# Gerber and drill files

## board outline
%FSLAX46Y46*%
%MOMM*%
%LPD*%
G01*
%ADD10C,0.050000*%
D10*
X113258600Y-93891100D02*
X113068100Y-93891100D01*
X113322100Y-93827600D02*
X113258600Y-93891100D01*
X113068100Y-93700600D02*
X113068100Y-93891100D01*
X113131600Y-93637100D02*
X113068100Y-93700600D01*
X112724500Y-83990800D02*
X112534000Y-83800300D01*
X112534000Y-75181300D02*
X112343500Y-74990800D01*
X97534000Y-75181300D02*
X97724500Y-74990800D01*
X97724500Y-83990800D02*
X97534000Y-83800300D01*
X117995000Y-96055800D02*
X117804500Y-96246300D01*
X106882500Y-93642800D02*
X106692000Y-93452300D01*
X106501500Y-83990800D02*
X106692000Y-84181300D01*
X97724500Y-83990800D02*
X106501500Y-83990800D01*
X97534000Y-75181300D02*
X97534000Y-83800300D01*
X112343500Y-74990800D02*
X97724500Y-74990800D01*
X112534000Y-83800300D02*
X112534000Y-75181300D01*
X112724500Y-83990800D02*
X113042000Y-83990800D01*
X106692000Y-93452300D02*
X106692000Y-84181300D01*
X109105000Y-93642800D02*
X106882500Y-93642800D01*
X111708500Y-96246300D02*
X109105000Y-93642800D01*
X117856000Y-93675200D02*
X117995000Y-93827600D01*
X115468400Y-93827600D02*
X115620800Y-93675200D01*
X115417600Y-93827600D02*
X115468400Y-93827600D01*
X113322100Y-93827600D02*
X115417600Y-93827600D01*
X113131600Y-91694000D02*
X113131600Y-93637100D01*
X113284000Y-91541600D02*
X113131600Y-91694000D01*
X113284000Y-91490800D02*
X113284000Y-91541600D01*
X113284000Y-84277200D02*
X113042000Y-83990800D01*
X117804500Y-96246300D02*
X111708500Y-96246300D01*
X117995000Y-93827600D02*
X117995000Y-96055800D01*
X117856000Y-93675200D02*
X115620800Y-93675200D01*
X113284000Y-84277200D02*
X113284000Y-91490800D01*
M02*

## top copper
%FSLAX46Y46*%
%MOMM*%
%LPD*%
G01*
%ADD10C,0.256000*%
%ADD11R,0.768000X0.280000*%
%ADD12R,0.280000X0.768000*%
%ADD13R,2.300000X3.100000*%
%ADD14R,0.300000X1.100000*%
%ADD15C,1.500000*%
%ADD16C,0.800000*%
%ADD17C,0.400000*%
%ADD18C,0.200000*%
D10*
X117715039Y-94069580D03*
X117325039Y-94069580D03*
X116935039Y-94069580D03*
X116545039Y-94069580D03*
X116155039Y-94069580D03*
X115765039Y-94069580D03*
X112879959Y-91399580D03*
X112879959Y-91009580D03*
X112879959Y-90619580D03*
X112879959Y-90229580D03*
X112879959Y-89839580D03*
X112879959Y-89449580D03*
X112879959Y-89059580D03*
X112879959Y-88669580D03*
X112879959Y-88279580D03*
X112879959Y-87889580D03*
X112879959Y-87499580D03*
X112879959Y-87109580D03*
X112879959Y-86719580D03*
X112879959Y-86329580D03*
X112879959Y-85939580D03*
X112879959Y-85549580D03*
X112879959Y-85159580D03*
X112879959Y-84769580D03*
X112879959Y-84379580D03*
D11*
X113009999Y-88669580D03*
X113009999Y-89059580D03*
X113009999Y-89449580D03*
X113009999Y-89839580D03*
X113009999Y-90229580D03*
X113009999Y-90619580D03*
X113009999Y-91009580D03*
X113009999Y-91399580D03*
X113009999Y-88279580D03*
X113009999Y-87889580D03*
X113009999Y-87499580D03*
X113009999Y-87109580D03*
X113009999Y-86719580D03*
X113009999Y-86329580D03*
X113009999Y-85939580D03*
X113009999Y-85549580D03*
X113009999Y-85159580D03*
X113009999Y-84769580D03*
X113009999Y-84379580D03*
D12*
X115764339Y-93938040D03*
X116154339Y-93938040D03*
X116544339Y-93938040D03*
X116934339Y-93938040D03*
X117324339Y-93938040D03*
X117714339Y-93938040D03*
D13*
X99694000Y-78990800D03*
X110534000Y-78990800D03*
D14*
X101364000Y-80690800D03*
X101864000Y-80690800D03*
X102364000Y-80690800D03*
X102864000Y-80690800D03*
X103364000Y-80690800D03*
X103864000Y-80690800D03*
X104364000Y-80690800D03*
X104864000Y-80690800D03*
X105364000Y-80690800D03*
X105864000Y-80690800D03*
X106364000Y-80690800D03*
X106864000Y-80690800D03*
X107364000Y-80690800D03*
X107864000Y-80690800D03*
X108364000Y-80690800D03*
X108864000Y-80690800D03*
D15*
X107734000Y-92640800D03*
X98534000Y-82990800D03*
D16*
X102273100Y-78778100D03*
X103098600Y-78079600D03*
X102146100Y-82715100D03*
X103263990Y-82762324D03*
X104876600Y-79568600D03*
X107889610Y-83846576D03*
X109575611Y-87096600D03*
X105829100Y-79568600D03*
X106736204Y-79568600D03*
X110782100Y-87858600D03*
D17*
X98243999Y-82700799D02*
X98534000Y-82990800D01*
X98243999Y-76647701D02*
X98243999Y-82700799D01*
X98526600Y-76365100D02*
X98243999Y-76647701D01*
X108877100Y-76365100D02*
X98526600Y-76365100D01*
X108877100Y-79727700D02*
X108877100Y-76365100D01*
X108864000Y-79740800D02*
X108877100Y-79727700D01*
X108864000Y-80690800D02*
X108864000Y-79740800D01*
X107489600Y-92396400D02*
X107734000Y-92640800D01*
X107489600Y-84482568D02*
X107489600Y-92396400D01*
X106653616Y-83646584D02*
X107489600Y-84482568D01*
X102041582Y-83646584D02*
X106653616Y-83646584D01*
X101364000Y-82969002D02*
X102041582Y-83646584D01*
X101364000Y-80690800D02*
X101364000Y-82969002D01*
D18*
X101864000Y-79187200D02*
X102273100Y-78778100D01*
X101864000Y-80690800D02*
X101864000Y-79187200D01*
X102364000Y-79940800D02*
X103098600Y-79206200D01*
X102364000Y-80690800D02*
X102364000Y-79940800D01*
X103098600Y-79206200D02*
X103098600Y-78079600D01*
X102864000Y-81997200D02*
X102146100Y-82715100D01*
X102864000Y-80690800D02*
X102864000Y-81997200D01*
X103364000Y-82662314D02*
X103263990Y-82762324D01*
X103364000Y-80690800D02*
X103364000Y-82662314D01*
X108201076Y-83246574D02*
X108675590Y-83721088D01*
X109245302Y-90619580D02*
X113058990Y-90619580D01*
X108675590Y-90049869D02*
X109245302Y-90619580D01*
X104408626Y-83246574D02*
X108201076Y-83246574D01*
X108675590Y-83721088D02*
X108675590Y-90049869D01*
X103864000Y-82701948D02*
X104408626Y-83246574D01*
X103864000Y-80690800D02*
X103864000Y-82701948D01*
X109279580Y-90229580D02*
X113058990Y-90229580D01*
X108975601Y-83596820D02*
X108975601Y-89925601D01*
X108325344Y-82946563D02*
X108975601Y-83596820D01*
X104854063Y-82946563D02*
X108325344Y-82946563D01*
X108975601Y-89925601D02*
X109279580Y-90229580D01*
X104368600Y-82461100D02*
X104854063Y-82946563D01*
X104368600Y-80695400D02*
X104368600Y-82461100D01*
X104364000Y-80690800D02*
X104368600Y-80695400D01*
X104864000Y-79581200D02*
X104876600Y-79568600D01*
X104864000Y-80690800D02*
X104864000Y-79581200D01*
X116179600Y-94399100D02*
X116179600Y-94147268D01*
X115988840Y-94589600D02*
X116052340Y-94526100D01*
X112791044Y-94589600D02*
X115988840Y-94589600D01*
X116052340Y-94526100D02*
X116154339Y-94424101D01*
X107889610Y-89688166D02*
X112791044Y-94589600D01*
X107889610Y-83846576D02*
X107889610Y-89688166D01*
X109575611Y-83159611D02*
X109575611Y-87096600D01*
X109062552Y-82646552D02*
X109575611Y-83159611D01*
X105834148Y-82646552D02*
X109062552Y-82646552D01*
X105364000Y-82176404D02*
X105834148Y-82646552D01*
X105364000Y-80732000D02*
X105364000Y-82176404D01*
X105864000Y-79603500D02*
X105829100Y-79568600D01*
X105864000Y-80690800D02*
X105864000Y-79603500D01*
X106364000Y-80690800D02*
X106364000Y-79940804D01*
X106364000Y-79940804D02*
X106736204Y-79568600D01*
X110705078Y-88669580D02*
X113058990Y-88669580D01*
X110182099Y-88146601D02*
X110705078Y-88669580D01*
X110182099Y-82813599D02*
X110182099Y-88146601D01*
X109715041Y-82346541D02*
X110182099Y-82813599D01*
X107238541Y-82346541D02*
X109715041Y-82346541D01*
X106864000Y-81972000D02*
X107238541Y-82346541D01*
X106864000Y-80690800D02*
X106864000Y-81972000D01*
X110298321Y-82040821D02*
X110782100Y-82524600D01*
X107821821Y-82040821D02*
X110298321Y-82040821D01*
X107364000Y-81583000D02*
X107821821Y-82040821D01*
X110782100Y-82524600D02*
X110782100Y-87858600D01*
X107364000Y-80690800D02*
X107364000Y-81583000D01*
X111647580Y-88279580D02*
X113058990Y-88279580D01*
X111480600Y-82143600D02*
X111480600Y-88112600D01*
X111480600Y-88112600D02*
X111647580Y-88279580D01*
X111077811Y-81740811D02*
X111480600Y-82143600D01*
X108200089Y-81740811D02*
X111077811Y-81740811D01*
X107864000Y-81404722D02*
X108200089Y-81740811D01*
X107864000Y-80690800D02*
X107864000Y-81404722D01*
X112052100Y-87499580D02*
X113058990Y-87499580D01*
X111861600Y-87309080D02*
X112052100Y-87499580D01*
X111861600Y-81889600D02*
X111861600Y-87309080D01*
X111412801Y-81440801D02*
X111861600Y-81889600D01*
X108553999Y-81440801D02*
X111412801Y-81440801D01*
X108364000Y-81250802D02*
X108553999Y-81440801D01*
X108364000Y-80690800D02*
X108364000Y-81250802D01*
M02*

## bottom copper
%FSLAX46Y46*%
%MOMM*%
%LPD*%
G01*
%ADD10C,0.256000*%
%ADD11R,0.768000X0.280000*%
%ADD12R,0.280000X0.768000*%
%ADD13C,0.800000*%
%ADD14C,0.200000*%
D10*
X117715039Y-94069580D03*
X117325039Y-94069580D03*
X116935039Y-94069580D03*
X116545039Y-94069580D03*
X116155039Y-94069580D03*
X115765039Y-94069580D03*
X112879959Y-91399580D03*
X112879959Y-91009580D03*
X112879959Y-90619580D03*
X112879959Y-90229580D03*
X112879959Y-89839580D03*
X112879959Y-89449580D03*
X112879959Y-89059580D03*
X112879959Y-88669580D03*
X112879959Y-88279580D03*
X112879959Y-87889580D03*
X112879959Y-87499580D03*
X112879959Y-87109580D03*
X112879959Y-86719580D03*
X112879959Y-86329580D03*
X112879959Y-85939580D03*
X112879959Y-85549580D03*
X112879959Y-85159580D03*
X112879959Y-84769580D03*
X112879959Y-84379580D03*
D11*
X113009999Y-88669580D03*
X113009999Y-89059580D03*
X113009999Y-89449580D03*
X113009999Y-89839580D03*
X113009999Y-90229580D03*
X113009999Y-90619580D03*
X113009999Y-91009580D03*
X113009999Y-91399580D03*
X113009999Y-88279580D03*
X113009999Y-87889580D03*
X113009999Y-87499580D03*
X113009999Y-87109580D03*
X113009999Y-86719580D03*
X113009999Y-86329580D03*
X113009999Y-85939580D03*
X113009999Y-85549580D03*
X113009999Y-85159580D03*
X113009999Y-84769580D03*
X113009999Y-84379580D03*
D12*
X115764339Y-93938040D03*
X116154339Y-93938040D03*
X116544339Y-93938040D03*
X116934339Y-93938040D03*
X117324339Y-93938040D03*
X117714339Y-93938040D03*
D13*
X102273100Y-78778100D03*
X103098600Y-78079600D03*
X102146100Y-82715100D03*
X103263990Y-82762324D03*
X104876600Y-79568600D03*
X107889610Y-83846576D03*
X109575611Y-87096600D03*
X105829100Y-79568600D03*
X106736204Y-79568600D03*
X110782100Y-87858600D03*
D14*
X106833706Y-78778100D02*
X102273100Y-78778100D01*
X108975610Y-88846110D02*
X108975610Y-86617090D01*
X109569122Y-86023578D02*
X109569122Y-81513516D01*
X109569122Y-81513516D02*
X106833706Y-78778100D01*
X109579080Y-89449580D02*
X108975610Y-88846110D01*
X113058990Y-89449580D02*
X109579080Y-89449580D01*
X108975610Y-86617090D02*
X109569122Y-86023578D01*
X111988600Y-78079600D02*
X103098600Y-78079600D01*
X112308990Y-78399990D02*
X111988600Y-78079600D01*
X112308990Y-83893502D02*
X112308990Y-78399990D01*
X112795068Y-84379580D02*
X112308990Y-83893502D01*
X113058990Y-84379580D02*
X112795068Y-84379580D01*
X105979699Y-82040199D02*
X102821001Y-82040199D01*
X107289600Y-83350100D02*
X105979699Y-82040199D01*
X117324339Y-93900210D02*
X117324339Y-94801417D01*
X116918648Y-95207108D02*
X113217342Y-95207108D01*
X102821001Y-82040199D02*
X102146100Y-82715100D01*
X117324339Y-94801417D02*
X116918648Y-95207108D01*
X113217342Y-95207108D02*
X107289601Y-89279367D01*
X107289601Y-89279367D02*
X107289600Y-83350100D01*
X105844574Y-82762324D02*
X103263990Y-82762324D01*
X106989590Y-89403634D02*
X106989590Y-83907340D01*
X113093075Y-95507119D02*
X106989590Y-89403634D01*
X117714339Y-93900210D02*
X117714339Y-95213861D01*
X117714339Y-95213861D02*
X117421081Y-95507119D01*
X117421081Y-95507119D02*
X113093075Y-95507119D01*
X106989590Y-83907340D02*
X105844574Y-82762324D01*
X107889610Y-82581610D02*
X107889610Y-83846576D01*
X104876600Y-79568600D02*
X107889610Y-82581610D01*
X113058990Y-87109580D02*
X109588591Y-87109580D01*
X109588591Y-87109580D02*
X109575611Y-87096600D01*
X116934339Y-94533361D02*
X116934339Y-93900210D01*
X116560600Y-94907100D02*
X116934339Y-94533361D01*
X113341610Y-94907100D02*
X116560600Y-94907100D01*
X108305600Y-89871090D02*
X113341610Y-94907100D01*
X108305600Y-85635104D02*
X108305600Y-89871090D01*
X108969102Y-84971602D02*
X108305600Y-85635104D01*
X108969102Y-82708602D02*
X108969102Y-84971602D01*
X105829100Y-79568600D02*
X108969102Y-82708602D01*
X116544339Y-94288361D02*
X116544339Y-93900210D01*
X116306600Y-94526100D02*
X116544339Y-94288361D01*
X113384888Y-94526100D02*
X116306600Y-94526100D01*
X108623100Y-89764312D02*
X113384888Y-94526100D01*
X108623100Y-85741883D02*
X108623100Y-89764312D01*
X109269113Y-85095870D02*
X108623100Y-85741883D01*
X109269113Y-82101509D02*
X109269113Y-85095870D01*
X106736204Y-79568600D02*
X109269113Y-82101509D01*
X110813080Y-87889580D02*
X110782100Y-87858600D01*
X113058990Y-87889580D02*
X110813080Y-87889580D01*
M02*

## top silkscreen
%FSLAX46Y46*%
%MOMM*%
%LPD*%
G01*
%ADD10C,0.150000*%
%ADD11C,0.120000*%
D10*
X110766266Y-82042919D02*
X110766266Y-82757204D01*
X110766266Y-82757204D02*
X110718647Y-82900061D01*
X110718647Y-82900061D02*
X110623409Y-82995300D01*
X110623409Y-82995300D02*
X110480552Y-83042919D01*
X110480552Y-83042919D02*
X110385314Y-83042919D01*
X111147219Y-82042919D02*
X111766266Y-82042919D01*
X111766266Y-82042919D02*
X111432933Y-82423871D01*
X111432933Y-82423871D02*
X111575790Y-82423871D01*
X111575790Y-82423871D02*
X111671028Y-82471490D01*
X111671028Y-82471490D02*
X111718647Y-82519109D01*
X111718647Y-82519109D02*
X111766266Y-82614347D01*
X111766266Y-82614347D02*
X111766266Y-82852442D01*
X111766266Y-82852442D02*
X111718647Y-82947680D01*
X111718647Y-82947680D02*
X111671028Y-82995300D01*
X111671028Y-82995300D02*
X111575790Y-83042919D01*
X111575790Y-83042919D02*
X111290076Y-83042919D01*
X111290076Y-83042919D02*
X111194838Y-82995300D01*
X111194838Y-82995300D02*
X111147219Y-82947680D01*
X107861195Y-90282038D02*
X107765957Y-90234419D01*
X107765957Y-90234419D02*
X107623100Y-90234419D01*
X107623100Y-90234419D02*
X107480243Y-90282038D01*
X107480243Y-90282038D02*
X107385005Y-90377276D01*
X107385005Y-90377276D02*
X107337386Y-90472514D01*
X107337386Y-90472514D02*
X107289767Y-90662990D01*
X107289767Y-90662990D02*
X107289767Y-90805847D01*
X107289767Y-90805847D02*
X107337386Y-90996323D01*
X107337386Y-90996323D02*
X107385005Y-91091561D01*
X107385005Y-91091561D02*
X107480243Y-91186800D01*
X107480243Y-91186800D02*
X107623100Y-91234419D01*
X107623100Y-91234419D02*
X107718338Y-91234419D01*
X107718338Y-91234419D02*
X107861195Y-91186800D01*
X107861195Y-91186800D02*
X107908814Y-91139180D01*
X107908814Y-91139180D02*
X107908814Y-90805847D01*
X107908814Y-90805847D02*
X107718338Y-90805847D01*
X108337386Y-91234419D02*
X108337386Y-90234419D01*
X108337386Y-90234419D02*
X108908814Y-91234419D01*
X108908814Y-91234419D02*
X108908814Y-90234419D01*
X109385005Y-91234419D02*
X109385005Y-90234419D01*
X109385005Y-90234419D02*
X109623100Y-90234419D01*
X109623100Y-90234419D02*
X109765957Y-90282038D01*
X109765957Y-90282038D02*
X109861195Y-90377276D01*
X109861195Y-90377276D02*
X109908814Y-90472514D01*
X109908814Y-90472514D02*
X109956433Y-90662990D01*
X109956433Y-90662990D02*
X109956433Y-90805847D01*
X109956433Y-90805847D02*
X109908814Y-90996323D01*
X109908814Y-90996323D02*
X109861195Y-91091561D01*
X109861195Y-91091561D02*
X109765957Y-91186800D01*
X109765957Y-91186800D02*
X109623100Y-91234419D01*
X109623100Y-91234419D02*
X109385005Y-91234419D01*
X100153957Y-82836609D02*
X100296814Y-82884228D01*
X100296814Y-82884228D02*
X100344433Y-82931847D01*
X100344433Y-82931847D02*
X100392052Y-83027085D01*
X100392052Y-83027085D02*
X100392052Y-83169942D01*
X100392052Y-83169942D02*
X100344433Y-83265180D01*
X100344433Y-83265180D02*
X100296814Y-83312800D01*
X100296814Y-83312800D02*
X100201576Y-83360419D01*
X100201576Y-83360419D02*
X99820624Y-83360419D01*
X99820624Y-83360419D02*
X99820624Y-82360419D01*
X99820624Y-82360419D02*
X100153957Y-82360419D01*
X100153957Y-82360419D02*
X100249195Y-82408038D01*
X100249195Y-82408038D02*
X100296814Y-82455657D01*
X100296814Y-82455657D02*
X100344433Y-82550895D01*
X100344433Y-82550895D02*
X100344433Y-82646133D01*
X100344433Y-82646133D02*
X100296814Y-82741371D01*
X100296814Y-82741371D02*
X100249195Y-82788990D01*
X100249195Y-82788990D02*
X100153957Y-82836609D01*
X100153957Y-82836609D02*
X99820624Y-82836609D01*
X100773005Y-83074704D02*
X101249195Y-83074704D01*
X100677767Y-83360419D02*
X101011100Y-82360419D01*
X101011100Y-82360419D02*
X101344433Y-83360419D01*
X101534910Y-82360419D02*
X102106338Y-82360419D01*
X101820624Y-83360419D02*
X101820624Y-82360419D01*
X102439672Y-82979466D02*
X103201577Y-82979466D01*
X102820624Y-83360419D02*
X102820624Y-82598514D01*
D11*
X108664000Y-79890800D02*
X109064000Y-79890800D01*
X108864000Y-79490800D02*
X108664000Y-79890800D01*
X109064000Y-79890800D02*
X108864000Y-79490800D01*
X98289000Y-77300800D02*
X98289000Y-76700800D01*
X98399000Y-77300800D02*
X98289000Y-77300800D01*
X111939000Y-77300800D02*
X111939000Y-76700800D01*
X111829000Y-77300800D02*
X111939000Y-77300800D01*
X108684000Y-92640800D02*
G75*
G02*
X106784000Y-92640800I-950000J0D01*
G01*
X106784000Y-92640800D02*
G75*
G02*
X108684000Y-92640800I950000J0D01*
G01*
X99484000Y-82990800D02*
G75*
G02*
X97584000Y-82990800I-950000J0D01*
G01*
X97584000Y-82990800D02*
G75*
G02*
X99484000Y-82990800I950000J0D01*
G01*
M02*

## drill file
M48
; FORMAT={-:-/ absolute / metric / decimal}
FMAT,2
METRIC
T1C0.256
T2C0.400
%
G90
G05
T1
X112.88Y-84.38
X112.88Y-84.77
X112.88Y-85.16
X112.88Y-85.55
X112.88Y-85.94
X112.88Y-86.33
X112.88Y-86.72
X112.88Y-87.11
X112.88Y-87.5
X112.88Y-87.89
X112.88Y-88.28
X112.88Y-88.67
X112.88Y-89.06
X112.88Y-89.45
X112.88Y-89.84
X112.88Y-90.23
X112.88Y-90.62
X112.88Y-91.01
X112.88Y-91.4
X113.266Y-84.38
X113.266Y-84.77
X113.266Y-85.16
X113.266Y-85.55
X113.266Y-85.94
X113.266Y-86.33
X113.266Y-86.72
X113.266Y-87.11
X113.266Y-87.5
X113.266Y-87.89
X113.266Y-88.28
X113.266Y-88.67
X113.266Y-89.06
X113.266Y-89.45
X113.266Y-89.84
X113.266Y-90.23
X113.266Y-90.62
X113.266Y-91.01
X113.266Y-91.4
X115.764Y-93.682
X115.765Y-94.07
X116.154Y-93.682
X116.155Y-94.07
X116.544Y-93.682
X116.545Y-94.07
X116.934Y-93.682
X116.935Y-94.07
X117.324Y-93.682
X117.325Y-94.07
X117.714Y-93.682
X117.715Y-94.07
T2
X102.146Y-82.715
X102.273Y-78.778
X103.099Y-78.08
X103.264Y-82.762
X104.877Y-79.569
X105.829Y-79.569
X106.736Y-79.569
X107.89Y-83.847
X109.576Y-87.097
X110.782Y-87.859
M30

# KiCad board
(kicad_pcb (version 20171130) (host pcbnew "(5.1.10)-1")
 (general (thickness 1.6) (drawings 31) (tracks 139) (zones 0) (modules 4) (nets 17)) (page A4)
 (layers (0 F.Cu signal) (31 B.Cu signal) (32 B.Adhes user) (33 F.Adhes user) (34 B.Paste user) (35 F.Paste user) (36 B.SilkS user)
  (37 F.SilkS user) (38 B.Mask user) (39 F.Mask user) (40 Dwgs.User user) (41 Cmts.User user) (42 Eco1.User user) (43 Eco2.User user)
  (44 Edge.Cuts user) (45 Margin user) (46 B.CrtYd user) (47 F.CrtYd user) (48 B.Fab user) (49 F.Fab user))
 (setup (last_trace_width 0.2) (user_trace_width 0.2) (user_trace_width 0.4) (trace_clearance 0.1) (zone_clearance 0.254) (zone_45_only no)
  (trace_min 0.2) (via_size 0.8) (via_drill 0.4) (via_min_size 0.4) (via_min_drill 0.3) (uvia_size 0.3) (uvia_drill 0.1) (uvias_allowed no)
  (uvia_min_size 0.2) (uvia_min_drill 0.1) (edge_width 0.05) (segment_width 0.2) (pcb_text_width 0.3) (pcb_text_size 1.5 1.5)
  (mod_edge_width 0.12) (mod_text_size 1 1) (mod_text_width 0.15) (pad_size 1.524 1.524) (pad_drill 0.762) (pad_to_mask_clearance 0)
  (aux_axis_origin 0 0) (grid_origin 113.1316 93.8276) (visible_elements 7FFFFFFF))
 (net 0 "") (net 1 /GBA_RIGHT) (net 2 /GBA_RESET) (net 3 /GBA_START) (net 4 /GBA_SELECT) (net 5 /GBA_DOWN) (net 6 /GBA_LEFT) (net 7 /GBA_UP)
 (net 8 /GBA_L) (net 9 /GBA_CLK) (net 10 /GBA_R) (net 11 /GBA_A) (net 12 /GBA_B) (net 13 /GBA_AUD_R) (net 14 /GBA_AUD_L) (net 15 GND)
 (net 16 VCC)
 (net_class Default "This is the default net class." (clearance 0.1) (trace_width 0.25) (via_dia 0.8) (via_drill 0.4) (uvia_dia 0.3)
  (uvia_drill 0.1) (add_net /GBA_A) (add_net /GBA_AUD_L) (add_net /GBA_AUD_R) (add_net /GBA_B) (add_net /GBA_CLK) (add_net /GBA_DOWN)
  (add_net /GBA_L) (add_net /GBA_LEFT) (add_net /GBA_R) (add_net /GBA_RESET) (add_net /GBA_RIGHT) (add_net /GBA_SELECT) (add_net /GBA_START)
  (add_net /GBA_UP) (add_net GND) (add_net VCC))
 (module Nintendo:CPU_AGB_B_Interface (layer F.Cu) (at 115.759959 89.84808)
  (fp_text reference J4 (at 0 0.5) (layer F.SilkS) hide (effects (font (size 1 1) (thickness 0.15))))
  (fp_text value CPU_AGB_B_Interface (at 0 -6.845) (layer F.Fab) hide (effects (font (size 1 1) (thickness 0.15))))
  (pad 0 thru_hole circle (at 1.95508 4.2215) (size 0.256 0.256) (drill 0.256) (layers *.Cu *.Mask))
  (pad 0 thru_hole circle (at 1.56508 4.2215) (size 0.256 0.256) (drill 0.256) (layers *.Cu *.Mask))
  (pad 0 thru_hole circle (at 1.17508 4.2215) (size 0.256 0.256) (drill 0.256) (layers *.Cu *.Mask))
  (pad 0 thru_hole circle (at 0.78508 4.2215) (size 0.256 0.256) (drill 0.256) (layers *.Cu *.Mask))
  (pad 0 thru_hole circle (at 0.39508 4.2215) (size 0.256 0.256) (drill 0.256) (layers *.Cu *.Mask))
  (pad 0 thru_hole circle (at 0.00508 4.2215) (size 0.256 0.256) (drill 0.256) (layers *.Cu *.Mask))
  (pad 0 thru_hole circle (at -2.88 1.5515) (size 0.256 0.256) (drill 0.256) (layers *.Cu *.Mask))
  (pad 0 thru_hole circle (at -2.88 1.1615) (size 0.256 0.256) (drill 0.256) (layers *.Cu *.Mask))
  (pad 0 thru_hole circle (at -2.88 0.7715) (size 0.256 0.256) (drill 0.256) (layers *.Cu *.Mask))
  (pad 0 thru_hole circle (at -2.88 0.3815) (size 0.256 0.256) (drill 0.256) (layers *.Cu *.Mask))
  (pad 0 thru_hole circle (at -2.88 -0.0085) (size 0.256 0.256) (drill 0.256) (layers *.Cu *.Mask))
  (pad 0 thru_hole circle (at -2.88 -0.3985) (size 0.256 0.256) (drill 0.256) (layers *.Cu *.Mask))
  (pad 0 thru_hole circle (at -2.88 -0.7885) (size 0.256 0.256) (drill 0.256) (layers *.Cu *.Mask))
  (pad 0 thru_hole circle (at -2.88 -1.1785) (size 0.256 0.256) (drill 0.256) (layers *.Cu *.Mask))
  (pad 0 thru_hole circle (at -2.88 -1.5685) (size 0.256 0.256) (drill 0.256) (layers *.Cu *.Mask))
  (pad 0 thru_hole circle (at -2.88 -1.9585) (size 0.256 0.256) (drill 0.256) (layers *.Cu *.Mask))
  (pad 0 thru_hole circle (at -2.88 -2.3485) (size 0.256 0.256) (drill 0.256) (layers *.Cu *.Mask))
  (pad 0 thru_hole circle (at -2.88 -2.7385) (size 0.256 0.256) (drill 0.256) (layers *.Cu *.Mask))
  (pad 0 thru_hole circle (at -2.88 -3.1285) (size 0.256 0.256) (drill 0.256) (layers *.Cu *.Mask))
  (pad 0 thru_hole circle (at -2.88 -3.5185) (size 0.256 0.256) (drill 0.256) (layers *.Cu *.Mask))
  (pad 0 thru_hole circle (at -2.88 -3.9085) (size 0.256 0.256) (drill 0.256) (layers *.Cu *.Mask))
  (pad 0 thru_hole circle (at -2.88 -4.2985) (size 0.256 0.256) (drill 0.256) (layers *.Cu *.Mask))
  (pad 0 thru_hole circle (at -2.88 -4.6885) (size 0.256 0.256) (drill 0.256) (layers *.Cu *.Mask))
  (pad 0 thru_hole circle (at -2.88 -5.0785) (size 0.256 0.256) (drill 0.256) (layers *.Cu *.Mask))
  (pad 0 thru_hole circle (at -2.88 -5.4685) (size 0.256 0.256) (drill 0.256) (layers *.Cu *.Mask))
  (pad 149 thru_hole rect (at -2.49396 -1.1785) (size 0.768 0.28) (drill 0.256 (offset -0.256 0)) (layers *.Cu *.Mask) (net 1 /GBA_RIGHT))
  (pad 150 thru_hole rect (at -2.49396 -0.7885) (size 0.768 0.28) (drill 0.256 (offset -0.256 0)) (layers *.Cu *.Mask))
  (pad 151 thru_hole rect (at -2.49396 -0.3985) (size 0.768 0.28) (drill 0.256 (offset -0.256 0)) (layers *.Cu *.Mask) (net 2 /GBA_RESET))
  (pad 152 thru_hole rect (at -2.49396 -0.0085) (size 0.768 0.28) (drill 0.256 (offset -0.256 0)) (layers *.Cu *.Mask))
  (pad 153 thru_hole rect (at -2.49396 0.3815) (size 0.768 0.28) (drill 0.256 (offset -0.256 0)) (layers *.Cu *.Mask) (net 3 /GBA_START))
  (pad 154 thru_hole rect (at -2.49396 0.7715) (size 0.768 0.28) (drill 0.256 (offset -0.256 0)) (layers *.Cu *.Mask) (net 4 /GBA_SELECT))
  (pad 155 thru_hole rect (at -2.49396 1.1615) (size 0.768 0.28) (drill 0.256 (offset -0.256 0)) (layers *.Cu *.Mask))
  (pad 156 thru_hole rect (at -2.49396 1.5515) (size 0.768 0.28) (drill 0.256 (offset -0.256 0)) (layers *.Cu *.Mask))
  (pad 148 thru_hole rect (at -2.49396 -1.5685) (size 0.768 0.28) (drill 0.256 (offset -0.256 0)) (layers *.Cu *.Mask) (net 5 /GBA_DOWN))
  (pad 147 thru_hole rect (at -2.49396 -1.9585) (size 0.768 0.28) (drill 0.256 (offset -0.256 0)) (layers *.Cu *.Mask) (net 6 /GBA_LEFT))
  (pad 146 thru_hole rect (at -2.49396 -2.3485) (size 0.768 0.28) (drill 0.256 (offset -0.256 0)) (layers *.Cu *.Mask) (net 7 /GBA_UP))
  (pad 145 thru_hole rect (at -2.49396 -2.7385) (size 0.768 0.28) (drill 0.256 (offset -0.256 0)) (layers *.Cu *.Mask) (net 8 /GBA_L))
  (pad 144 thru_hole rect (at -2.49396 -3.1285) (size 0.768 0.28) (drill 0.256 (offset -0.256 0)) (layers *.Cu *.Mask))
  (pad 143 thru_hole rect (at -2.49396 -3.5185) (size 0.768 0.28) (drill 0.256 (offset -0.256 0)) (layers *.Cu *.Mask))
  (pad 142 thru_hole rect (at -2.49396 -3.9085) (size 0.768 0.28) (drill 0.256 (offset -0.256 0)) (layers *.Cu *.Mask))
  (pad 141 thru_hole rect (at -2.49396 -4.2985) (size 0.768 0.28) (drill 0.256 (offset -0.256 0)) (layers *.Cu *.Mask))
  (pad 140 thru_hole rect (at -2.49396 -4.6885) (size 0.768 0.28) (drill 0.256 (offset -0.256 0)) (layers *.Cu *.Mask))
  (pad 139 thru_hole rect (at -2.49396 -5.0785) (size 0.768 0.28) (drill 0.256 (offset -0.256 0)) (layers *.Cu *.Mask))
  (pad 138 thru_hole rect (at -2.49396 -5.4685) (size 0.768 0.28) (drill 0.256 (offset -0.256 0)) (layers *.Cu *.Mask) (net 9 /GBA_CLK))
  (pad 1 thru_hole rect (at 0.00438 3.83396 90) (size 0.768 0.28) (drill 0.256 (offset -0.256 0)) (layers *.Cu *.Mask))
  (pad 2 thru_hole rect (at 0.39438 3.83396 90) (size 0.768 0.28) (drill 0.256 (offset -0.256 0)) (layers *.Cu *.Mask) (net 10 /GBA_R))
  (pad 3 thru_hole rect (at 0.78438 3.83396 90) (size 0.768 0.28) (drill 0.256 (offset -0.256 0)) (layers *.Cu *.Mask) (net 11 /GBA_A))
  (pad 4 thru_hole rect (at 1.17438 3.83396 90) (size 0.768 0.28) (drill 0.256 (offset -0.256 0)) (layers *.Cu *.Mask) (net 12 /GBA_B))
  (pad 5 thru_hole rect (at 1.56438 3.83396 90) (size 0.768 0.28) (drill 0.256 (offset -0.256 0)) (layers *.Cu *.Mask) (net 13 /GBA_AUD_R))
  (pad 6 thru_hole rect (at 1.95438 3.83396 90) (size 0.768 0.28) (drill 0.256 (offset -0.256 0)) (layers *.Cu *.Mask) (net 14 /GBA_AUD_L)))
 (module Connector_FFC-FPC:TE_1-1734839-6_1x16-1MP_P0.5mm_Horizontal (layer F.Cu) (at 105.114 79.3408 180)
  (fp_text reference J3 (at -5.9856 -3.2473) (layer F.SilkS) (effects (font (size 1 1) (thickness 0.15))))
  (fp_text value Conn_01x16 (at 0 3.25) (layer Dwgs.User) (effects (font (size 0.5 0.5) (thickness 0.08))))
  (fp_line (start -3.55 -0.55) (end -3.95 -0.55) (layer F.SilkS) (width 0.12))
  (fp_line (start -3.75 -0.15) (end -3.55 -0.55) (layer F.SilkS) (width 0.12))
  (fp_line (start -3.95 -0.55) (end -3.75 -0.15) (layer F.SilkS) (width 0.12))
  (fp_line (start 6.825 2.04) (end 6.825 2.64) (layer F.SilkS) (width 0.12))
  (fp_line (start 6.715 2.04) (end 6.825 2.04) (layer F.SilkS) (width 0.12))
  (fp_line (start -6.825 2.04) (end -6.825 2.64) (layer F.SilkS) (width 0.12))
  (fp_line (start -6.715 2.04) (end -6.825 2.04) (layer F.SilkS) (width 0.12))
  (pad MP smd rect (at 5.42 0.35 180) (size 2.3 3.1) (layers F.Cu F.Paste F.Mask))
  (pad MP smd rect (at -5.42 0.35 180) (size 2.3 3.1) (layers F.Cu F.Paste F.Mask))
  (pad 16 smd rect (at 3.75 -1.35 180) (size 0.3 1.1) (layers F.Cu F.Paste F.Mask) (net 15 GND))
  (pad 15 smd rect (at 3.25 -1.35 180) (size 0.3 1.1) (layers F.Cu F.Paste F.Mask) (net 2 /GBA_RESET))
  (pad 14 smd rect (at 2.75 -1.35 180) (size 0.3 1.1) (layers F.Cu F.Paste F.Mask) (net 9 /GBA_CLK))
  (pad 13 smd rect (at 2.25 -1.35 180) (size 0.3 1.1) (layers F.Cu F.Paste F.Mask) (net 13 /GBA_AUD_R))
  (pad 12 smd rect (at 1.75 -1.35 180) (size 0.3 1.1) (layers F.Cu F.Paste F.Mask) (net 14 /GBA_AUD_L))
  (pad 11 smd rect (at 1.25 -1.35 180) (size 0.3 1.1) (layers F.Cu F.Paste F.Mask) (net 4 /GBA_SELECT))
  (pad 10 smd rect (at 0.75 -1.35 180) (size 0.3 1.1) (layers F.Cu F.Paste F.Mask) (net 3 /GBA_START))
  (pad 9 smd rect (at 0.25 -1.35 180) (size 0.3 1.1) (layers F.Cu F.Paste F.Mask) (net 10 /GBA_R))
  (pad 8 smd rect (at -0.25 -1.35 180) (size 0.3 1.1) (layers F.Cu F.Paste F.Mask) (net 8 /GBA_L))
  (pad 7 smd rect (at -0.75 -1.35 180) (size 0.3 1.1) (layers F.Cu F.Paste F.Mask) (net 12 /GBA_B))
  (pad 6 smd rect (at -1.25 -1.35 180) (size 0.3 1.1) (layers F.Cu F.Paste F.Mask) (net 11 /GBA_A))
  (pad 5 smd rect (at -1.75 -1.35 180) (size 0.3 1.1) (layers F.Cu F.Paste F.Mask) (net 1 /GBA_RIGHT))
  (pad 4 smd rect (at -2.25 -1.35 180) (size 0.3 1.1) (layers F.Cu F.Paste F.Mask) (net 6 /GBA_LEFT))
  (pad 3 smd rect (at -2.75 -1.35 180) (size 0.3 1.1) (layers F.Cu F.Paste F.Mask) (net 5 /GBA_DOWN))
  (pad 2 smd rect (at -3.25 -1.35 180) (size 0.3 1.1) (layers F.Cu F.Paste F.Mask) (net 7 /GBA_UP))
  (pad 1 smd rect (at -3.75 -1.35 180) (size 0.3 1.1) (layers F.Cu F.Paste F.Mask) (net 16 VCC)))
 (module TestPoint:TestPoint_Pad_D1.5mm (layer F.Cu) (at 107.734 92.6408)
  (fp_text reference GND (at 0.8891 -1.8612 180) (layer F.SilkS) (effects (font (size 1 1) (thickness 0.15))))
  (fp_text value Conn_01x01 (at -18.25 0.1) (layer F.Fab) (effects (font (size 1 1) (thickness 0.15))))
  (fp_circle (center 0 0) (end 0 0.95) (layer F.SilkS) (width 0.12))
  (pad 1 smd circle (at 0 0) (size 1.5 1.5) (layers F.Cu F.Mask) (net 15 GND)))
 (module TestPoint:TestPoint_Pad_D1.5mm (layer F.Cu) (at 98.534 82.9908)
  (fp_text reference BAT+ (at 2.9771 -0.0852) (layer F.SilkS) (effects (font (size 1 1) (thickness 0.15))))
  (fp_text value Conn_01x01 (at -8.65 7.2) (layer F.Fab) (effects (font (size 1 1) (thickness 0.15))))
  (fp_circle (center 0 0) (end 0 0.95) (layer F.SilkS) (width 0.12))
  (pad 1 smd circle (at 0 0) (size 1.5 1.5) (layers F.Cu F.Mask) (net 16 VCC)))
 (gr_line (start 113.2586 93.8911) (end 113.0681 93.8911) (layer Edge.Cuts) (width 0.05))
 (gr_line (start 113.3221 93.8276) (end 113.2586 93.8911) (layer Edge.Cuts) (width 0.05))
 (gr_line (start 113.0681 93.7006) (end 113.0681 93.8911) (layer Edge.Cuts) (width 0.05))
 (gr_line (start 113.1316 93.6371) (end 113.0681 93.7006) (layer Edge.Cuts) (width 0.05))
 (gr_line (start 112.7245 83.9908) (end 112.534 83.8003) (layer Edge.Cuts) (width 0.05))
 (gr_line (start 112.534 75.1813) (end 112.3435 74.9908) (layer Edge.Cuts) (width 0.05))
 (gr_line (start 97.534 75.1813) (end 97.7245 74.9908) (layer Edge.Cuts) (width 0.05))
 (gr_line (start 97.7245 83.9908) (end 97.534 83.8003) (layer Edge.Cuts) (width 0.05))
 (gr_line (start 117.995 96.0558) (end 117.8045 96.2463) (layer Edge.Cuts) (width 0.05))
 (gr_line (start 106.8825 93.6428) (end 106.692 93.4523) (layer Edge.Cuts) (width 0.05))
 (gr_line (start 106.5015 83.9908) (end 106.692 84.1813) (layer Edge.Cuts) (width 0.05))
 (gr_line (start 97.7245 83.9908) (end 106.5015 83.9908) (layer Edge.Cuts) (width 0.05))
 (gr_line (start 97.534 75.1813) (end 97.534 83.8003) (layer Edge.Cuts) (width 0.05))
 (gr_line (start 112.3435 74.9908) (end 97.7245 74.9908) (layer Edge.Cuts) (width 0.05))
 (gr_line (start 112.534 83.8003) (end 112.534 75.1813) (layer Edge.Cuts) (width 0.05))
 (gr_line (start 112.7245 83.9908) (end 113.042 83.9908) (layer Edge.Cuts) (width 0.05))
 (gr_line (start 106.692 93.4523) (end 106.692 84.1813) (layer Edge.Cuts) (width 0.05))
 (gr_line (start 109.105 93.6428) (end 106.8825 93.6428) (layer Edge.Cuts) (width 0.05))
 (gr_line (start 111.7085 96.2463) (end 109.105 93.6428) (layer Edge.Cuts) (width 0.05))
 (gr_line (start 117.856 93.6752) (end 117.995 93.8276) (layer Edge.Cuts) (width 0.05))
 (gr_line (start 115.4684 93.8276) (end 115.6208 93.6752) (layer Edge.Cuts) (width 0.05))
 (gr_line (start 115.4176 93.8276) (end 115.4684 93.8276) (layer Edge.Cuts) (width 0.05))
 (gr_line (start 113.3221 93.8276) (end 115.4176 93.8276) (layer Edge.Cuts) (width 0.05))
 (gr_line (start 113.1316 91.694) (end 113.1316 93.6371) (layer Edge.Cuts) (width 0.05))
 (gr_line (start 113.284 91.5416) (end 113.1316 91.694) (layer Edge.Cuts) (width 0.05))
 (gr_line (start 113.284 91.4908) (end 113.284 91.5416) (layer Edge.Cuts) (width 0.05))
 (gr_line (start 113.284 84.2772) (end 113.042 83.9908) (layer Edge.Cuts) (width 0.05))
 (gr_line (start 117.8045 96.2463) (end 111.7085 96.2463) (layer Edge.Cuts) (width 0.05))
 (gr_line (start 117.995 93.8276) (end 117.995 96.0558) (layer Edge.Cuts) (width 0.05))
 (gr_line (start 117.856 93.6752) (end 115.6208 93.6752) (layer Edge.Cuts) (width 0.05))
 (gr_line (start 113.284 84.2772) (end 113.284 91.4908) (layer Edge.Cuts) (width 0.05))
 (segment (start 98.243999 82.700799) (end 98.534 82.9908) (width 0.4) (layer F.Cu) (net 16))
 (segment (start 98.243999 76.647701) (end 98.243999 82.700799) (width 0.4) (layer F.Cu) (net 16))
 (segment (start 98.5266 76.3651) (end 98.243999 76.647701) (width 0.4) (layer F.Cu) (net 16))
 (segment (start 108.8771 76.3651) (end 98.5266 76.3651) (width 0.4) (layer F.Cu) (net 16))
 (segment (start 108.8771 79.7277) (end 108.8771 76.3651) (width 0.4) (layer F.Cu) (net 16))
 (segment (start 108.864 79.7408) (end 108.8771 79.7277) (width 0.4) (layer F.Cu) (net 16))
 (segment (start 108.864 80.6908) (end 108.864 79.7408) (width 0.4) (layer F.Cu) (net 16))
 (segment (start 107.4896 92.3964) (end 107.734 92.6408) (width 0.4) (layer F.Cu) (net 15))
 (segment (start 107.4896 84.482568) (end 107.4896 92.3964) (width 0.4) (layer F.Cu) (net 15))
 (segment (start 106.653616 83.646584) (end 107.4896 84.482568) (width 0.4) (layer F.Cu) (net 15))
 (segment (start 102.041582 83.646584) (end 106.653616 83.646584) (width 0.4) (layer F.Cu) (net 15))
 (segment (start 101.364 82.969002) (end 102.041582 83.646584) (width 0.4) (layer F.Cu) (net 15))
 (segment (start 101.364 80.6908) (end 101.364 82.969002) (width 0.4) (layer F.Cu) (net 15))
 (segment (start 106.833706 78.7781) (end 102.2731 78.7781) (width 0.2) (layer B.Cu) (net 2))
 (segment (start 101.864 79.1872) (end 102.2731 78.7781) (width 0.2) (layer F.Cu) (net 2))
 (segment (start 108.97561 88.84611) (end 108.97561 86.61709) (width 0.2) (layer B.Cu) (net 2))
 (segment (start 109.569122 86.023578) (end 109.569122 81.513516) (width 0.2) (layer B.Cu) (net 2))
 (via (at 102.2731 78.7781) (size 0.8) (drill 0.4) (layers F.Cu B.Cu) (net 2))
 (segment (start 109.569122 81.513516) (end 106.833706 78.7781) (width 0.2) (layer B.Cu) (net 2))
 (segment (start 101.864 80.6908) (end 101.864 79.1872) (width 0.2) (layer F.Cu) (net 2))
 (segment (start 109.57908 89.44958) (end 108.97561 88.84611) (width 0.2) (layer B.Cu) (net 2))
 (segment (start 113.05899 89.44958) (end 109.57908 89.44958) (width 0.2) (layer B.Cu) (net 2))
 (segment (start 108.97561 86.61709) (end 109.569122 86.023578) (width 0.2) (layer B.Cu) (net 2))
 (segment (start 111.9886 78.0796) (end 103.0986 78.0796) (width 0.2) (layer B.Cu) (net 9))
 (segment (start 112.30899 78.39999) (end 111.9886 78.0796) (width 0.2) (layer B.Cu) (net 9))
 (segment (start 112.30899 83.893502) (end 112.30899 78.39999) (width 0.2) (layer B.Cu) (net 9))
 (segment (start 112.795068 84.37958) (end 112.30899 83.893502) (width 0.2) (layer B.Cu) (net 9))
 (segment (start 113.05899 84.37958) (end 112.795068 84.37958) (width 0.2) (layer B.Cu) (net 9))
 (via (at 103.0986 78.0796) (size 0.8) (drill 0.4) (layers F.Cu B.Cu) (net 9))
 (segment (start 102.364 79.9408) (end 103.0986 79.2062) (width 0.2) (layer F.Cu) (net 9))
 (segment (start 102.364 80.6908) (end 102.364 79.9408) (width 0.2) (layer F.Cu) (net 9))
 (segment (start 103.0986 79.2062) (end 103.0986 78.0796) (width 0.2) (layer F.Cu) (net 9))
 (via (at 102.1461 82.7151) (size 0.8) (drill 0.4) (layers F.Cu B.Cu) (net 13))
 (segment (start 102.864 81.9972) (end 102.1461 82.7151) (width 0.2) (layer F.Cu) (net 13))
 (segment (start 102.864 80.6908) (end 102.864 81.9972) (width 0.2) (layer F.Cu) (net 13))
 (segment (start 105.979699 82.040199) (end 102.821001 82.040199) (width 0.2) (layer B.Cu) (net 13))
 (segment (start 107.2896 83.3501) (end 105.979699 82.040199) (width 0.2) (layer B.Cu) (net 13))
 (segment (start 117.324339 93.90021) (end 117.324339 94.801417) (width 0.2) (layer B.Cu) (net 13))
 (segment (start 116.918648 95.207108) (end 113.217342 95.207108) (width 0.2) (layer B.Cu) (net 13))
 (segment (start 102.821001 82.040199) (end 102.1461 82.7151) (width 0.2) (layer B.Cu) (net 13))
 (segment (start 117.324339 94.801417) (end 116.918648 95.207108) (width 0.2) (layer B.Cu) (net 13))
 (segment (start 113.217342 95.207108) (end 107.289601 89.279367) (width 0.2) (layer B.Cu) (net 13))
 (segment (start 107.289601 89.279367) (end 107.2896 83.3501) (width 0.2) (layer B.Cu) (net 13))
 (segment (start 105.844574 82.762324) (end 103.26399 82.762324) (width 0.2) (layer B.Cu) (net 14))
 (segment (start 103.364 82.662314) (end 103.26399 82.762324) (width 0.2) (layer F.Cu) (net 14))
 (segment (start 106.98959 89.403634) (end 106.98959 83.90734) (width 0.2) (layer B.Cu) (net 14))
 (via (at 103.26399 82.762324) (size 0.8) (drill 0.4) (layers F.Cu B.Cu) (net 14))
 (segment (start 113.093075 95.507119) (end 106.98959 89.403634) (width 0.2) (layer B.Cu) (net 14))
 (segment (start 117.714339 93.90021) (end 117.714339 95.213861) (width 0.2) (layer B.Cu) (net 14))
 (segment (start 117.714339 95.213861) (end 117.421081 95.507119) (width 0.2) (layer B.Cu) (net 14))
 (segment (start 103.364 80.6908) (end 103.364 82.662314) (width 0.2) (layer F.Cu) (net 14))
 (segment (start 117.421081 95.507119) (end 113.093075 95.507119) (width 0.2) (layer B.Cu) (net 14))
 (segment (start 106.98959 83.90734) (end 105.844574 82.762324) (width 0.2) (layer B.Cu) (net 14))
 (segment (start 108.201076 83.246574) (end 108.67559 83.721088) (width 0.2) (layer F.Cu) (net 4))
 (segment (start 109.245302 90.61958) (end 113.05899 90.61958) (width 0.2) (layer F.Cu) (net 4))
 (segment (start 108.67559 90.049869) (end 109.245302 90.61958) (width 0.2) (layer F.Cu) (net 4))
 (segment (start 104.408626 83.246574) (end 108.201076 83.246574) (width 0.2) (layer F.Cu) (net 4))
 (segment (start 108.67559 83.721088) (end 108.67559 90.049869) (width 0.2) (layer F.Cu) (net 4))
 (segment (start 103.864 82.701948) (end 104.408626 83.246574) (width 0.2) (layer F.Cu) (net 4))
 (segment (start 103.864 80.6908) (end 103.864 82.701948) (width 0.2) (layer F.Cu) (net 4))
 (segment (start 109.27958 90.22958) (end 113.05899 90.22958) (width 0.2) (layer F.Cu) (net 3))
 (segment (start 108.975601 83.59682) (end 108.975601 89.925601) (width 0.2) (layer F.Cu) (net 3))
 (segment (start 108.325344 82.946563) (end 108.975601 83.59682) (width 0.2) (layer F.Cu) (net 3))
 (segment (start 104.854063 82.946563) (end 108.325344 82.946563) (width 0.2) (layer F.Cu) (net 3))
 (segment (start 108.975601 89.925601) (end 109.27958 90.22958) (width 0.2) (layer F.Cu) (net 3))
 (segment (start 104.3686 82.4611) (end 104.854063 82.946563) (width 0.2) (layer F.Cu) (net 3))
 (segment (start 104.3686 80.6954) (end 104.3686 82.4611) (width 0.2) (layer F.Cu) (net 3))
 (segment (start 104.364 80.6908) (end 104.3686 80.6954) (width 0.2) (layer F.Cu) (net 3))
 (via (at 104.8766 79.5686) (size 0.8) (drill 0.4) (layers F.Cu B.Cu) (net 10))
 (segment (start 104.864 79.5812) (end 104.8766 79.5686) (width 0.2) (layer F.Cu) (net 10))
 (segment (start 104.864 80.6908) (end 104.864 79.5812) (width 0.2) (layer F.Cu) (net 10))
 (segment (start 116.1796 94.3991) (end 116.1796 94.147268) (width 0.2) (layer F.Cu) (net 10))
 (segment (start 107.88961 82.58161) (end 107.88961 83.846576) (width 0.2) (layer B.Cu) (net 10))
 (segment (start 104.8766 79.5686) (end 107.88961 82.58161) (width 0.2) (layer B.Cu) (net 10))
 (via (at 107.88961 83.846576) (size 0.8) (drill 0.4) (layers F.Cu B.Cu) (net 10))
 (segment (start 115.98884 94.5896) (end 116.05234 94.5261) (width 0.2) (layer F.Cu) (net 10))
 (segment (start 112.791044 94.5896) (end 115.98884 94.5896) (width 0.2) (layer F.Cu) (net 10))
 (segment (start 116.05234 94.5261) (end 116.154339 94.424101) (width 0.2) (layer F.Cu) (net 10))
 (segment (start 107.88961 89.688166) (end 112.791044 94.5896) (width 0.2) (layer F.Cu) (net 10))
 (segment (start 107.88961 83.846576) (end 107.88961 89.688166) (width 0.2) (layer F.Cu) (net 10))
 (via (at 109.575611 87.0966) (size 0.8) (drill 0.4) (layers F.Cu B.Cu) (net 8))
 (segment (start 113.05899 87.10958) (end 109.588591 87.10958) (width 0.2) (layer B.Cu) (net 8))
 (segment (start 109.588591 87.10958) (end 109.575611 87.0966) (width 0.2) (layer B.Cu) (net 8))
 (segment (start 109.575611 83.159611) (end 109.575611 87.0966) (width 0.2) (layer F.Cu) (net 8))
 (segment (start 109.062552 82.646552) (end 109.575611 83.159611) (width 0.2) (layer F.Cu) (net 8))
 (segment (start 105.834148 82.646552) (end 109.062552 82.646552) (width 0.2) (layer F.Cu) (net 8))
 (segment (start 105.364 82.176404) (end 105.834148 82.646552) (width 0.2) (layer F.Cu) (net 8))
 (segment (start 105.364 80.732) (end 105.364 82.176404) (width 0.2) (layer F.Cu) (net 8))
 (via (at 105.8291 79.5686) (size 0.8) (drill 0.4) (layers F.Cu B.Cu) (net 12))
 (segment (start 105.864 79.6035) (end 105.8291 79.5686) (width 0.2) (layer F.Cu) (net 12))
 (segment (start 105.864 80.6908) (end 105.864 79.6035) (width 0.2) (layer F.Cu) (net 12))
 (segment (start 116.934339 94.533361) (end 116.934339 93.90021) (width 0.2) (layer B.Cu) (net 12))
 (segment (start 116.5606 94.9071) (end 116.934339 94.533361) (width 0.2) (layer B.Cu) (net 12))
 (segment (start 113.34161 94.9071) (end 116.5606 94.9071) (width 0.2) (layer B.Cu) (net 12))
 (segment (start 108.3056 89.87109) (end 113.34161 94.9071) (width 0.2) (layer B.Cu) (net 12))
 (segment (start 108.3056 85.635104) (end 108.3056 89.87109) (width 0.2) (layer B.Cu) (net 12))
 (segment (start 108.969102 84.971602) (end 108.3056 85.635104) (width 0.2) (layer B.Cu) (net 12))
 (segment (start 108.969102 82.708602) (end 108.969102 84.971602) (width 0.2) (layer B.Cu) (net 12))
 (segment (start 105.8291 79.5686) (end 108.969102 82.708602) (width 0.2) (layer B.Cu) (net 12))
 (via (at 106.736204 79.5686) (size 0.8) (drill 0.4) (layers F.Cu B.Cu) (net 11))
 (segment (start 106.364 80.6908) (end 106.364 79.940804) (width 0.2) (layer F.Cu) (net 11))
 (segment (start 106.364 79.940804) (end 106.736204 79.5686) (width 0.2) (layer F.Cu) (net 11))
 (segment (start 116.544339 94.288361) (end 116.544339 93.90021) (width 0.2) (layer B.Cu) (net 11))
 (segment (start 116.3066 94.5261) (end 116.544339 94.288361) (width 0.2) (layer B.Cu) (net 11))
 (segment (start 113.384888 94.5261) (end 116.3066 94.5261) (width 0.2) (layer B.Cu) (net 11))
 (segment (start 108.6231 89.764312) (end 113.384888 94.5261) (width 0.2) (layer B.Cu) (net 11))
 (segment (start 108.6231 85.741883) (end 108.6231 89.764312) (width 0.2) (layer B.Cu) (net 11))
 (segment (start 109.269113 85.09587) (end 108.6231 85.741883) (width 0.2) (layer B.Cu) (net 11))
 (segment (start 109.269113 82.101509) (end 109.269113 85.09587) (width 0.2) (layer B.Cu) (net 11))
 (segment (start 106.736204 79.5686) (end 109.269113 82.101509) (width 0.2) (layer B.Cu) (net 11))
 (segment (start 110.705078 88.66958) (end 113.05899 88.66958) (width 0.2) (layer F.Cu) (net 1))
 (segment (start 110.182099 88.146601) (end 110.705078 88.66958) (width 0.2) (layer F.Cu) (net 1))
 (segment (start 110.182099 82.813599) (end 110.182099 88.146601) (width 0.2) (layer F.Cu) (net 1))
 (segment (start 109.715041 82.346541) (end 110.182099 82.813599) (width 0.2) (layer F.Cu) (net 1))
 (segment (start 107.238541 82.346541) (end 109.715041 82.346541) (width 0.2) (layer F.Cu) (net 1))
 (segment (start 106.864 81.972) (end 107.238541 82.346541) (width 0.2) (layer F.Cu) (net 1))
 (segment (start 106.864 80.6908) (end 106.864 81.972) (width 0.2) (layer F.Cu) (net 1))
 (segment (start 110.81308 87.88958) (end 110.7821 87.8586) (width 0.2) (layer B.Cu) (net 6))
 (segment (start 113.05899 87.88958) (end 110.81308 87.88958) (width 0.2) (layer B.Cu) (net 6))
 (via (at 110.7821 87.8586) (size 0.8) (drill 0.4) (layers F.Cu B.Cu) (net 6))
 (segment (start 110.298321 82.040821) (end 110.7821 82.5246) (width 0.2) (layer F.Cu) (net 6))
 (segment (start 107.821821 82.040821) (end 110.298321 82.040821) (width 0.2) (layer F.Cu) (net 6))
 (segment (start 107.364 81.583) (end 107.821821 82.040821) (width 0.2) (layer F.Cu) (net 6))
 (segment (start 110.7821 82.5246) (end 110.7821 87.8586) (width 0.2) (layer F.Cu) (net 6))
 (segment (start 107.364 80.6908) (end 107.364 81.583) (width 0.2) (layer F.Cu) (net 6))
 (segment (start 111.64758 88.27958) (end 113.05899 88.27958) (width 0.2) (layer F.Cu) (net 5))
 (segment (start 111.4806 82.1436) (end 111.4806 88.1126) (width 0.2) (layer F.Cu) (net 5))
 (segment (start 111.4806 88.1126) (end 111.64758 88.27958) (width 0.2) (layer F.Cu) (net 5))
 (segment (start 111.077811 81.740811) (end 111.4806 82.1436) (width 0.2) (layer F.Cu) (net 5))
 (segment (start 108.200089 81.740811) (end 111.077811 81.740811) (width 0.2) (layer F.Cu) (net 5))
 (segment (start 107.864 81.404722) (end 108.200089 81.740811) (width 0.2) (layer F.Cu) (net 5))
 (segment (start 107.864 80.6908) (end 107.864 81.404722) (width 0.2) (layer F.Cu) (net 5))
 (segment (start 112.0521 87.49958) (end 113.05899 87.49958) (width 0.2) (layer F.Cu) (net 7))
 (segment (start 111.8616 87.30908) (end 112.0521 87.49958) (width 0.2) (layer F.Cu) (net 7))
 (segment (start 111.8616 81.8896) (end 111.8616 87.30908) (width 0.2) (layer F.Cu) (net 7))
 (segment (start 111.412801 81.440801) (end 111.8616 81.8896) (width 0.2) (layer F.Cu) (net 7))
 (segment (start 108.553999 81.440801) (end 111.412801 81.440801) (width 0.2) (layer F.Cu) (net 7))
 (segment (start 108.364 81.250802) (end 108.553999 81.440801) (width 0.2) (layer F.Cu) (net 7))
 (segment (start 108.364 80.6908) (end 108.364 81.250802) (width 0.2) (layer F.Cu) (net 7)))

